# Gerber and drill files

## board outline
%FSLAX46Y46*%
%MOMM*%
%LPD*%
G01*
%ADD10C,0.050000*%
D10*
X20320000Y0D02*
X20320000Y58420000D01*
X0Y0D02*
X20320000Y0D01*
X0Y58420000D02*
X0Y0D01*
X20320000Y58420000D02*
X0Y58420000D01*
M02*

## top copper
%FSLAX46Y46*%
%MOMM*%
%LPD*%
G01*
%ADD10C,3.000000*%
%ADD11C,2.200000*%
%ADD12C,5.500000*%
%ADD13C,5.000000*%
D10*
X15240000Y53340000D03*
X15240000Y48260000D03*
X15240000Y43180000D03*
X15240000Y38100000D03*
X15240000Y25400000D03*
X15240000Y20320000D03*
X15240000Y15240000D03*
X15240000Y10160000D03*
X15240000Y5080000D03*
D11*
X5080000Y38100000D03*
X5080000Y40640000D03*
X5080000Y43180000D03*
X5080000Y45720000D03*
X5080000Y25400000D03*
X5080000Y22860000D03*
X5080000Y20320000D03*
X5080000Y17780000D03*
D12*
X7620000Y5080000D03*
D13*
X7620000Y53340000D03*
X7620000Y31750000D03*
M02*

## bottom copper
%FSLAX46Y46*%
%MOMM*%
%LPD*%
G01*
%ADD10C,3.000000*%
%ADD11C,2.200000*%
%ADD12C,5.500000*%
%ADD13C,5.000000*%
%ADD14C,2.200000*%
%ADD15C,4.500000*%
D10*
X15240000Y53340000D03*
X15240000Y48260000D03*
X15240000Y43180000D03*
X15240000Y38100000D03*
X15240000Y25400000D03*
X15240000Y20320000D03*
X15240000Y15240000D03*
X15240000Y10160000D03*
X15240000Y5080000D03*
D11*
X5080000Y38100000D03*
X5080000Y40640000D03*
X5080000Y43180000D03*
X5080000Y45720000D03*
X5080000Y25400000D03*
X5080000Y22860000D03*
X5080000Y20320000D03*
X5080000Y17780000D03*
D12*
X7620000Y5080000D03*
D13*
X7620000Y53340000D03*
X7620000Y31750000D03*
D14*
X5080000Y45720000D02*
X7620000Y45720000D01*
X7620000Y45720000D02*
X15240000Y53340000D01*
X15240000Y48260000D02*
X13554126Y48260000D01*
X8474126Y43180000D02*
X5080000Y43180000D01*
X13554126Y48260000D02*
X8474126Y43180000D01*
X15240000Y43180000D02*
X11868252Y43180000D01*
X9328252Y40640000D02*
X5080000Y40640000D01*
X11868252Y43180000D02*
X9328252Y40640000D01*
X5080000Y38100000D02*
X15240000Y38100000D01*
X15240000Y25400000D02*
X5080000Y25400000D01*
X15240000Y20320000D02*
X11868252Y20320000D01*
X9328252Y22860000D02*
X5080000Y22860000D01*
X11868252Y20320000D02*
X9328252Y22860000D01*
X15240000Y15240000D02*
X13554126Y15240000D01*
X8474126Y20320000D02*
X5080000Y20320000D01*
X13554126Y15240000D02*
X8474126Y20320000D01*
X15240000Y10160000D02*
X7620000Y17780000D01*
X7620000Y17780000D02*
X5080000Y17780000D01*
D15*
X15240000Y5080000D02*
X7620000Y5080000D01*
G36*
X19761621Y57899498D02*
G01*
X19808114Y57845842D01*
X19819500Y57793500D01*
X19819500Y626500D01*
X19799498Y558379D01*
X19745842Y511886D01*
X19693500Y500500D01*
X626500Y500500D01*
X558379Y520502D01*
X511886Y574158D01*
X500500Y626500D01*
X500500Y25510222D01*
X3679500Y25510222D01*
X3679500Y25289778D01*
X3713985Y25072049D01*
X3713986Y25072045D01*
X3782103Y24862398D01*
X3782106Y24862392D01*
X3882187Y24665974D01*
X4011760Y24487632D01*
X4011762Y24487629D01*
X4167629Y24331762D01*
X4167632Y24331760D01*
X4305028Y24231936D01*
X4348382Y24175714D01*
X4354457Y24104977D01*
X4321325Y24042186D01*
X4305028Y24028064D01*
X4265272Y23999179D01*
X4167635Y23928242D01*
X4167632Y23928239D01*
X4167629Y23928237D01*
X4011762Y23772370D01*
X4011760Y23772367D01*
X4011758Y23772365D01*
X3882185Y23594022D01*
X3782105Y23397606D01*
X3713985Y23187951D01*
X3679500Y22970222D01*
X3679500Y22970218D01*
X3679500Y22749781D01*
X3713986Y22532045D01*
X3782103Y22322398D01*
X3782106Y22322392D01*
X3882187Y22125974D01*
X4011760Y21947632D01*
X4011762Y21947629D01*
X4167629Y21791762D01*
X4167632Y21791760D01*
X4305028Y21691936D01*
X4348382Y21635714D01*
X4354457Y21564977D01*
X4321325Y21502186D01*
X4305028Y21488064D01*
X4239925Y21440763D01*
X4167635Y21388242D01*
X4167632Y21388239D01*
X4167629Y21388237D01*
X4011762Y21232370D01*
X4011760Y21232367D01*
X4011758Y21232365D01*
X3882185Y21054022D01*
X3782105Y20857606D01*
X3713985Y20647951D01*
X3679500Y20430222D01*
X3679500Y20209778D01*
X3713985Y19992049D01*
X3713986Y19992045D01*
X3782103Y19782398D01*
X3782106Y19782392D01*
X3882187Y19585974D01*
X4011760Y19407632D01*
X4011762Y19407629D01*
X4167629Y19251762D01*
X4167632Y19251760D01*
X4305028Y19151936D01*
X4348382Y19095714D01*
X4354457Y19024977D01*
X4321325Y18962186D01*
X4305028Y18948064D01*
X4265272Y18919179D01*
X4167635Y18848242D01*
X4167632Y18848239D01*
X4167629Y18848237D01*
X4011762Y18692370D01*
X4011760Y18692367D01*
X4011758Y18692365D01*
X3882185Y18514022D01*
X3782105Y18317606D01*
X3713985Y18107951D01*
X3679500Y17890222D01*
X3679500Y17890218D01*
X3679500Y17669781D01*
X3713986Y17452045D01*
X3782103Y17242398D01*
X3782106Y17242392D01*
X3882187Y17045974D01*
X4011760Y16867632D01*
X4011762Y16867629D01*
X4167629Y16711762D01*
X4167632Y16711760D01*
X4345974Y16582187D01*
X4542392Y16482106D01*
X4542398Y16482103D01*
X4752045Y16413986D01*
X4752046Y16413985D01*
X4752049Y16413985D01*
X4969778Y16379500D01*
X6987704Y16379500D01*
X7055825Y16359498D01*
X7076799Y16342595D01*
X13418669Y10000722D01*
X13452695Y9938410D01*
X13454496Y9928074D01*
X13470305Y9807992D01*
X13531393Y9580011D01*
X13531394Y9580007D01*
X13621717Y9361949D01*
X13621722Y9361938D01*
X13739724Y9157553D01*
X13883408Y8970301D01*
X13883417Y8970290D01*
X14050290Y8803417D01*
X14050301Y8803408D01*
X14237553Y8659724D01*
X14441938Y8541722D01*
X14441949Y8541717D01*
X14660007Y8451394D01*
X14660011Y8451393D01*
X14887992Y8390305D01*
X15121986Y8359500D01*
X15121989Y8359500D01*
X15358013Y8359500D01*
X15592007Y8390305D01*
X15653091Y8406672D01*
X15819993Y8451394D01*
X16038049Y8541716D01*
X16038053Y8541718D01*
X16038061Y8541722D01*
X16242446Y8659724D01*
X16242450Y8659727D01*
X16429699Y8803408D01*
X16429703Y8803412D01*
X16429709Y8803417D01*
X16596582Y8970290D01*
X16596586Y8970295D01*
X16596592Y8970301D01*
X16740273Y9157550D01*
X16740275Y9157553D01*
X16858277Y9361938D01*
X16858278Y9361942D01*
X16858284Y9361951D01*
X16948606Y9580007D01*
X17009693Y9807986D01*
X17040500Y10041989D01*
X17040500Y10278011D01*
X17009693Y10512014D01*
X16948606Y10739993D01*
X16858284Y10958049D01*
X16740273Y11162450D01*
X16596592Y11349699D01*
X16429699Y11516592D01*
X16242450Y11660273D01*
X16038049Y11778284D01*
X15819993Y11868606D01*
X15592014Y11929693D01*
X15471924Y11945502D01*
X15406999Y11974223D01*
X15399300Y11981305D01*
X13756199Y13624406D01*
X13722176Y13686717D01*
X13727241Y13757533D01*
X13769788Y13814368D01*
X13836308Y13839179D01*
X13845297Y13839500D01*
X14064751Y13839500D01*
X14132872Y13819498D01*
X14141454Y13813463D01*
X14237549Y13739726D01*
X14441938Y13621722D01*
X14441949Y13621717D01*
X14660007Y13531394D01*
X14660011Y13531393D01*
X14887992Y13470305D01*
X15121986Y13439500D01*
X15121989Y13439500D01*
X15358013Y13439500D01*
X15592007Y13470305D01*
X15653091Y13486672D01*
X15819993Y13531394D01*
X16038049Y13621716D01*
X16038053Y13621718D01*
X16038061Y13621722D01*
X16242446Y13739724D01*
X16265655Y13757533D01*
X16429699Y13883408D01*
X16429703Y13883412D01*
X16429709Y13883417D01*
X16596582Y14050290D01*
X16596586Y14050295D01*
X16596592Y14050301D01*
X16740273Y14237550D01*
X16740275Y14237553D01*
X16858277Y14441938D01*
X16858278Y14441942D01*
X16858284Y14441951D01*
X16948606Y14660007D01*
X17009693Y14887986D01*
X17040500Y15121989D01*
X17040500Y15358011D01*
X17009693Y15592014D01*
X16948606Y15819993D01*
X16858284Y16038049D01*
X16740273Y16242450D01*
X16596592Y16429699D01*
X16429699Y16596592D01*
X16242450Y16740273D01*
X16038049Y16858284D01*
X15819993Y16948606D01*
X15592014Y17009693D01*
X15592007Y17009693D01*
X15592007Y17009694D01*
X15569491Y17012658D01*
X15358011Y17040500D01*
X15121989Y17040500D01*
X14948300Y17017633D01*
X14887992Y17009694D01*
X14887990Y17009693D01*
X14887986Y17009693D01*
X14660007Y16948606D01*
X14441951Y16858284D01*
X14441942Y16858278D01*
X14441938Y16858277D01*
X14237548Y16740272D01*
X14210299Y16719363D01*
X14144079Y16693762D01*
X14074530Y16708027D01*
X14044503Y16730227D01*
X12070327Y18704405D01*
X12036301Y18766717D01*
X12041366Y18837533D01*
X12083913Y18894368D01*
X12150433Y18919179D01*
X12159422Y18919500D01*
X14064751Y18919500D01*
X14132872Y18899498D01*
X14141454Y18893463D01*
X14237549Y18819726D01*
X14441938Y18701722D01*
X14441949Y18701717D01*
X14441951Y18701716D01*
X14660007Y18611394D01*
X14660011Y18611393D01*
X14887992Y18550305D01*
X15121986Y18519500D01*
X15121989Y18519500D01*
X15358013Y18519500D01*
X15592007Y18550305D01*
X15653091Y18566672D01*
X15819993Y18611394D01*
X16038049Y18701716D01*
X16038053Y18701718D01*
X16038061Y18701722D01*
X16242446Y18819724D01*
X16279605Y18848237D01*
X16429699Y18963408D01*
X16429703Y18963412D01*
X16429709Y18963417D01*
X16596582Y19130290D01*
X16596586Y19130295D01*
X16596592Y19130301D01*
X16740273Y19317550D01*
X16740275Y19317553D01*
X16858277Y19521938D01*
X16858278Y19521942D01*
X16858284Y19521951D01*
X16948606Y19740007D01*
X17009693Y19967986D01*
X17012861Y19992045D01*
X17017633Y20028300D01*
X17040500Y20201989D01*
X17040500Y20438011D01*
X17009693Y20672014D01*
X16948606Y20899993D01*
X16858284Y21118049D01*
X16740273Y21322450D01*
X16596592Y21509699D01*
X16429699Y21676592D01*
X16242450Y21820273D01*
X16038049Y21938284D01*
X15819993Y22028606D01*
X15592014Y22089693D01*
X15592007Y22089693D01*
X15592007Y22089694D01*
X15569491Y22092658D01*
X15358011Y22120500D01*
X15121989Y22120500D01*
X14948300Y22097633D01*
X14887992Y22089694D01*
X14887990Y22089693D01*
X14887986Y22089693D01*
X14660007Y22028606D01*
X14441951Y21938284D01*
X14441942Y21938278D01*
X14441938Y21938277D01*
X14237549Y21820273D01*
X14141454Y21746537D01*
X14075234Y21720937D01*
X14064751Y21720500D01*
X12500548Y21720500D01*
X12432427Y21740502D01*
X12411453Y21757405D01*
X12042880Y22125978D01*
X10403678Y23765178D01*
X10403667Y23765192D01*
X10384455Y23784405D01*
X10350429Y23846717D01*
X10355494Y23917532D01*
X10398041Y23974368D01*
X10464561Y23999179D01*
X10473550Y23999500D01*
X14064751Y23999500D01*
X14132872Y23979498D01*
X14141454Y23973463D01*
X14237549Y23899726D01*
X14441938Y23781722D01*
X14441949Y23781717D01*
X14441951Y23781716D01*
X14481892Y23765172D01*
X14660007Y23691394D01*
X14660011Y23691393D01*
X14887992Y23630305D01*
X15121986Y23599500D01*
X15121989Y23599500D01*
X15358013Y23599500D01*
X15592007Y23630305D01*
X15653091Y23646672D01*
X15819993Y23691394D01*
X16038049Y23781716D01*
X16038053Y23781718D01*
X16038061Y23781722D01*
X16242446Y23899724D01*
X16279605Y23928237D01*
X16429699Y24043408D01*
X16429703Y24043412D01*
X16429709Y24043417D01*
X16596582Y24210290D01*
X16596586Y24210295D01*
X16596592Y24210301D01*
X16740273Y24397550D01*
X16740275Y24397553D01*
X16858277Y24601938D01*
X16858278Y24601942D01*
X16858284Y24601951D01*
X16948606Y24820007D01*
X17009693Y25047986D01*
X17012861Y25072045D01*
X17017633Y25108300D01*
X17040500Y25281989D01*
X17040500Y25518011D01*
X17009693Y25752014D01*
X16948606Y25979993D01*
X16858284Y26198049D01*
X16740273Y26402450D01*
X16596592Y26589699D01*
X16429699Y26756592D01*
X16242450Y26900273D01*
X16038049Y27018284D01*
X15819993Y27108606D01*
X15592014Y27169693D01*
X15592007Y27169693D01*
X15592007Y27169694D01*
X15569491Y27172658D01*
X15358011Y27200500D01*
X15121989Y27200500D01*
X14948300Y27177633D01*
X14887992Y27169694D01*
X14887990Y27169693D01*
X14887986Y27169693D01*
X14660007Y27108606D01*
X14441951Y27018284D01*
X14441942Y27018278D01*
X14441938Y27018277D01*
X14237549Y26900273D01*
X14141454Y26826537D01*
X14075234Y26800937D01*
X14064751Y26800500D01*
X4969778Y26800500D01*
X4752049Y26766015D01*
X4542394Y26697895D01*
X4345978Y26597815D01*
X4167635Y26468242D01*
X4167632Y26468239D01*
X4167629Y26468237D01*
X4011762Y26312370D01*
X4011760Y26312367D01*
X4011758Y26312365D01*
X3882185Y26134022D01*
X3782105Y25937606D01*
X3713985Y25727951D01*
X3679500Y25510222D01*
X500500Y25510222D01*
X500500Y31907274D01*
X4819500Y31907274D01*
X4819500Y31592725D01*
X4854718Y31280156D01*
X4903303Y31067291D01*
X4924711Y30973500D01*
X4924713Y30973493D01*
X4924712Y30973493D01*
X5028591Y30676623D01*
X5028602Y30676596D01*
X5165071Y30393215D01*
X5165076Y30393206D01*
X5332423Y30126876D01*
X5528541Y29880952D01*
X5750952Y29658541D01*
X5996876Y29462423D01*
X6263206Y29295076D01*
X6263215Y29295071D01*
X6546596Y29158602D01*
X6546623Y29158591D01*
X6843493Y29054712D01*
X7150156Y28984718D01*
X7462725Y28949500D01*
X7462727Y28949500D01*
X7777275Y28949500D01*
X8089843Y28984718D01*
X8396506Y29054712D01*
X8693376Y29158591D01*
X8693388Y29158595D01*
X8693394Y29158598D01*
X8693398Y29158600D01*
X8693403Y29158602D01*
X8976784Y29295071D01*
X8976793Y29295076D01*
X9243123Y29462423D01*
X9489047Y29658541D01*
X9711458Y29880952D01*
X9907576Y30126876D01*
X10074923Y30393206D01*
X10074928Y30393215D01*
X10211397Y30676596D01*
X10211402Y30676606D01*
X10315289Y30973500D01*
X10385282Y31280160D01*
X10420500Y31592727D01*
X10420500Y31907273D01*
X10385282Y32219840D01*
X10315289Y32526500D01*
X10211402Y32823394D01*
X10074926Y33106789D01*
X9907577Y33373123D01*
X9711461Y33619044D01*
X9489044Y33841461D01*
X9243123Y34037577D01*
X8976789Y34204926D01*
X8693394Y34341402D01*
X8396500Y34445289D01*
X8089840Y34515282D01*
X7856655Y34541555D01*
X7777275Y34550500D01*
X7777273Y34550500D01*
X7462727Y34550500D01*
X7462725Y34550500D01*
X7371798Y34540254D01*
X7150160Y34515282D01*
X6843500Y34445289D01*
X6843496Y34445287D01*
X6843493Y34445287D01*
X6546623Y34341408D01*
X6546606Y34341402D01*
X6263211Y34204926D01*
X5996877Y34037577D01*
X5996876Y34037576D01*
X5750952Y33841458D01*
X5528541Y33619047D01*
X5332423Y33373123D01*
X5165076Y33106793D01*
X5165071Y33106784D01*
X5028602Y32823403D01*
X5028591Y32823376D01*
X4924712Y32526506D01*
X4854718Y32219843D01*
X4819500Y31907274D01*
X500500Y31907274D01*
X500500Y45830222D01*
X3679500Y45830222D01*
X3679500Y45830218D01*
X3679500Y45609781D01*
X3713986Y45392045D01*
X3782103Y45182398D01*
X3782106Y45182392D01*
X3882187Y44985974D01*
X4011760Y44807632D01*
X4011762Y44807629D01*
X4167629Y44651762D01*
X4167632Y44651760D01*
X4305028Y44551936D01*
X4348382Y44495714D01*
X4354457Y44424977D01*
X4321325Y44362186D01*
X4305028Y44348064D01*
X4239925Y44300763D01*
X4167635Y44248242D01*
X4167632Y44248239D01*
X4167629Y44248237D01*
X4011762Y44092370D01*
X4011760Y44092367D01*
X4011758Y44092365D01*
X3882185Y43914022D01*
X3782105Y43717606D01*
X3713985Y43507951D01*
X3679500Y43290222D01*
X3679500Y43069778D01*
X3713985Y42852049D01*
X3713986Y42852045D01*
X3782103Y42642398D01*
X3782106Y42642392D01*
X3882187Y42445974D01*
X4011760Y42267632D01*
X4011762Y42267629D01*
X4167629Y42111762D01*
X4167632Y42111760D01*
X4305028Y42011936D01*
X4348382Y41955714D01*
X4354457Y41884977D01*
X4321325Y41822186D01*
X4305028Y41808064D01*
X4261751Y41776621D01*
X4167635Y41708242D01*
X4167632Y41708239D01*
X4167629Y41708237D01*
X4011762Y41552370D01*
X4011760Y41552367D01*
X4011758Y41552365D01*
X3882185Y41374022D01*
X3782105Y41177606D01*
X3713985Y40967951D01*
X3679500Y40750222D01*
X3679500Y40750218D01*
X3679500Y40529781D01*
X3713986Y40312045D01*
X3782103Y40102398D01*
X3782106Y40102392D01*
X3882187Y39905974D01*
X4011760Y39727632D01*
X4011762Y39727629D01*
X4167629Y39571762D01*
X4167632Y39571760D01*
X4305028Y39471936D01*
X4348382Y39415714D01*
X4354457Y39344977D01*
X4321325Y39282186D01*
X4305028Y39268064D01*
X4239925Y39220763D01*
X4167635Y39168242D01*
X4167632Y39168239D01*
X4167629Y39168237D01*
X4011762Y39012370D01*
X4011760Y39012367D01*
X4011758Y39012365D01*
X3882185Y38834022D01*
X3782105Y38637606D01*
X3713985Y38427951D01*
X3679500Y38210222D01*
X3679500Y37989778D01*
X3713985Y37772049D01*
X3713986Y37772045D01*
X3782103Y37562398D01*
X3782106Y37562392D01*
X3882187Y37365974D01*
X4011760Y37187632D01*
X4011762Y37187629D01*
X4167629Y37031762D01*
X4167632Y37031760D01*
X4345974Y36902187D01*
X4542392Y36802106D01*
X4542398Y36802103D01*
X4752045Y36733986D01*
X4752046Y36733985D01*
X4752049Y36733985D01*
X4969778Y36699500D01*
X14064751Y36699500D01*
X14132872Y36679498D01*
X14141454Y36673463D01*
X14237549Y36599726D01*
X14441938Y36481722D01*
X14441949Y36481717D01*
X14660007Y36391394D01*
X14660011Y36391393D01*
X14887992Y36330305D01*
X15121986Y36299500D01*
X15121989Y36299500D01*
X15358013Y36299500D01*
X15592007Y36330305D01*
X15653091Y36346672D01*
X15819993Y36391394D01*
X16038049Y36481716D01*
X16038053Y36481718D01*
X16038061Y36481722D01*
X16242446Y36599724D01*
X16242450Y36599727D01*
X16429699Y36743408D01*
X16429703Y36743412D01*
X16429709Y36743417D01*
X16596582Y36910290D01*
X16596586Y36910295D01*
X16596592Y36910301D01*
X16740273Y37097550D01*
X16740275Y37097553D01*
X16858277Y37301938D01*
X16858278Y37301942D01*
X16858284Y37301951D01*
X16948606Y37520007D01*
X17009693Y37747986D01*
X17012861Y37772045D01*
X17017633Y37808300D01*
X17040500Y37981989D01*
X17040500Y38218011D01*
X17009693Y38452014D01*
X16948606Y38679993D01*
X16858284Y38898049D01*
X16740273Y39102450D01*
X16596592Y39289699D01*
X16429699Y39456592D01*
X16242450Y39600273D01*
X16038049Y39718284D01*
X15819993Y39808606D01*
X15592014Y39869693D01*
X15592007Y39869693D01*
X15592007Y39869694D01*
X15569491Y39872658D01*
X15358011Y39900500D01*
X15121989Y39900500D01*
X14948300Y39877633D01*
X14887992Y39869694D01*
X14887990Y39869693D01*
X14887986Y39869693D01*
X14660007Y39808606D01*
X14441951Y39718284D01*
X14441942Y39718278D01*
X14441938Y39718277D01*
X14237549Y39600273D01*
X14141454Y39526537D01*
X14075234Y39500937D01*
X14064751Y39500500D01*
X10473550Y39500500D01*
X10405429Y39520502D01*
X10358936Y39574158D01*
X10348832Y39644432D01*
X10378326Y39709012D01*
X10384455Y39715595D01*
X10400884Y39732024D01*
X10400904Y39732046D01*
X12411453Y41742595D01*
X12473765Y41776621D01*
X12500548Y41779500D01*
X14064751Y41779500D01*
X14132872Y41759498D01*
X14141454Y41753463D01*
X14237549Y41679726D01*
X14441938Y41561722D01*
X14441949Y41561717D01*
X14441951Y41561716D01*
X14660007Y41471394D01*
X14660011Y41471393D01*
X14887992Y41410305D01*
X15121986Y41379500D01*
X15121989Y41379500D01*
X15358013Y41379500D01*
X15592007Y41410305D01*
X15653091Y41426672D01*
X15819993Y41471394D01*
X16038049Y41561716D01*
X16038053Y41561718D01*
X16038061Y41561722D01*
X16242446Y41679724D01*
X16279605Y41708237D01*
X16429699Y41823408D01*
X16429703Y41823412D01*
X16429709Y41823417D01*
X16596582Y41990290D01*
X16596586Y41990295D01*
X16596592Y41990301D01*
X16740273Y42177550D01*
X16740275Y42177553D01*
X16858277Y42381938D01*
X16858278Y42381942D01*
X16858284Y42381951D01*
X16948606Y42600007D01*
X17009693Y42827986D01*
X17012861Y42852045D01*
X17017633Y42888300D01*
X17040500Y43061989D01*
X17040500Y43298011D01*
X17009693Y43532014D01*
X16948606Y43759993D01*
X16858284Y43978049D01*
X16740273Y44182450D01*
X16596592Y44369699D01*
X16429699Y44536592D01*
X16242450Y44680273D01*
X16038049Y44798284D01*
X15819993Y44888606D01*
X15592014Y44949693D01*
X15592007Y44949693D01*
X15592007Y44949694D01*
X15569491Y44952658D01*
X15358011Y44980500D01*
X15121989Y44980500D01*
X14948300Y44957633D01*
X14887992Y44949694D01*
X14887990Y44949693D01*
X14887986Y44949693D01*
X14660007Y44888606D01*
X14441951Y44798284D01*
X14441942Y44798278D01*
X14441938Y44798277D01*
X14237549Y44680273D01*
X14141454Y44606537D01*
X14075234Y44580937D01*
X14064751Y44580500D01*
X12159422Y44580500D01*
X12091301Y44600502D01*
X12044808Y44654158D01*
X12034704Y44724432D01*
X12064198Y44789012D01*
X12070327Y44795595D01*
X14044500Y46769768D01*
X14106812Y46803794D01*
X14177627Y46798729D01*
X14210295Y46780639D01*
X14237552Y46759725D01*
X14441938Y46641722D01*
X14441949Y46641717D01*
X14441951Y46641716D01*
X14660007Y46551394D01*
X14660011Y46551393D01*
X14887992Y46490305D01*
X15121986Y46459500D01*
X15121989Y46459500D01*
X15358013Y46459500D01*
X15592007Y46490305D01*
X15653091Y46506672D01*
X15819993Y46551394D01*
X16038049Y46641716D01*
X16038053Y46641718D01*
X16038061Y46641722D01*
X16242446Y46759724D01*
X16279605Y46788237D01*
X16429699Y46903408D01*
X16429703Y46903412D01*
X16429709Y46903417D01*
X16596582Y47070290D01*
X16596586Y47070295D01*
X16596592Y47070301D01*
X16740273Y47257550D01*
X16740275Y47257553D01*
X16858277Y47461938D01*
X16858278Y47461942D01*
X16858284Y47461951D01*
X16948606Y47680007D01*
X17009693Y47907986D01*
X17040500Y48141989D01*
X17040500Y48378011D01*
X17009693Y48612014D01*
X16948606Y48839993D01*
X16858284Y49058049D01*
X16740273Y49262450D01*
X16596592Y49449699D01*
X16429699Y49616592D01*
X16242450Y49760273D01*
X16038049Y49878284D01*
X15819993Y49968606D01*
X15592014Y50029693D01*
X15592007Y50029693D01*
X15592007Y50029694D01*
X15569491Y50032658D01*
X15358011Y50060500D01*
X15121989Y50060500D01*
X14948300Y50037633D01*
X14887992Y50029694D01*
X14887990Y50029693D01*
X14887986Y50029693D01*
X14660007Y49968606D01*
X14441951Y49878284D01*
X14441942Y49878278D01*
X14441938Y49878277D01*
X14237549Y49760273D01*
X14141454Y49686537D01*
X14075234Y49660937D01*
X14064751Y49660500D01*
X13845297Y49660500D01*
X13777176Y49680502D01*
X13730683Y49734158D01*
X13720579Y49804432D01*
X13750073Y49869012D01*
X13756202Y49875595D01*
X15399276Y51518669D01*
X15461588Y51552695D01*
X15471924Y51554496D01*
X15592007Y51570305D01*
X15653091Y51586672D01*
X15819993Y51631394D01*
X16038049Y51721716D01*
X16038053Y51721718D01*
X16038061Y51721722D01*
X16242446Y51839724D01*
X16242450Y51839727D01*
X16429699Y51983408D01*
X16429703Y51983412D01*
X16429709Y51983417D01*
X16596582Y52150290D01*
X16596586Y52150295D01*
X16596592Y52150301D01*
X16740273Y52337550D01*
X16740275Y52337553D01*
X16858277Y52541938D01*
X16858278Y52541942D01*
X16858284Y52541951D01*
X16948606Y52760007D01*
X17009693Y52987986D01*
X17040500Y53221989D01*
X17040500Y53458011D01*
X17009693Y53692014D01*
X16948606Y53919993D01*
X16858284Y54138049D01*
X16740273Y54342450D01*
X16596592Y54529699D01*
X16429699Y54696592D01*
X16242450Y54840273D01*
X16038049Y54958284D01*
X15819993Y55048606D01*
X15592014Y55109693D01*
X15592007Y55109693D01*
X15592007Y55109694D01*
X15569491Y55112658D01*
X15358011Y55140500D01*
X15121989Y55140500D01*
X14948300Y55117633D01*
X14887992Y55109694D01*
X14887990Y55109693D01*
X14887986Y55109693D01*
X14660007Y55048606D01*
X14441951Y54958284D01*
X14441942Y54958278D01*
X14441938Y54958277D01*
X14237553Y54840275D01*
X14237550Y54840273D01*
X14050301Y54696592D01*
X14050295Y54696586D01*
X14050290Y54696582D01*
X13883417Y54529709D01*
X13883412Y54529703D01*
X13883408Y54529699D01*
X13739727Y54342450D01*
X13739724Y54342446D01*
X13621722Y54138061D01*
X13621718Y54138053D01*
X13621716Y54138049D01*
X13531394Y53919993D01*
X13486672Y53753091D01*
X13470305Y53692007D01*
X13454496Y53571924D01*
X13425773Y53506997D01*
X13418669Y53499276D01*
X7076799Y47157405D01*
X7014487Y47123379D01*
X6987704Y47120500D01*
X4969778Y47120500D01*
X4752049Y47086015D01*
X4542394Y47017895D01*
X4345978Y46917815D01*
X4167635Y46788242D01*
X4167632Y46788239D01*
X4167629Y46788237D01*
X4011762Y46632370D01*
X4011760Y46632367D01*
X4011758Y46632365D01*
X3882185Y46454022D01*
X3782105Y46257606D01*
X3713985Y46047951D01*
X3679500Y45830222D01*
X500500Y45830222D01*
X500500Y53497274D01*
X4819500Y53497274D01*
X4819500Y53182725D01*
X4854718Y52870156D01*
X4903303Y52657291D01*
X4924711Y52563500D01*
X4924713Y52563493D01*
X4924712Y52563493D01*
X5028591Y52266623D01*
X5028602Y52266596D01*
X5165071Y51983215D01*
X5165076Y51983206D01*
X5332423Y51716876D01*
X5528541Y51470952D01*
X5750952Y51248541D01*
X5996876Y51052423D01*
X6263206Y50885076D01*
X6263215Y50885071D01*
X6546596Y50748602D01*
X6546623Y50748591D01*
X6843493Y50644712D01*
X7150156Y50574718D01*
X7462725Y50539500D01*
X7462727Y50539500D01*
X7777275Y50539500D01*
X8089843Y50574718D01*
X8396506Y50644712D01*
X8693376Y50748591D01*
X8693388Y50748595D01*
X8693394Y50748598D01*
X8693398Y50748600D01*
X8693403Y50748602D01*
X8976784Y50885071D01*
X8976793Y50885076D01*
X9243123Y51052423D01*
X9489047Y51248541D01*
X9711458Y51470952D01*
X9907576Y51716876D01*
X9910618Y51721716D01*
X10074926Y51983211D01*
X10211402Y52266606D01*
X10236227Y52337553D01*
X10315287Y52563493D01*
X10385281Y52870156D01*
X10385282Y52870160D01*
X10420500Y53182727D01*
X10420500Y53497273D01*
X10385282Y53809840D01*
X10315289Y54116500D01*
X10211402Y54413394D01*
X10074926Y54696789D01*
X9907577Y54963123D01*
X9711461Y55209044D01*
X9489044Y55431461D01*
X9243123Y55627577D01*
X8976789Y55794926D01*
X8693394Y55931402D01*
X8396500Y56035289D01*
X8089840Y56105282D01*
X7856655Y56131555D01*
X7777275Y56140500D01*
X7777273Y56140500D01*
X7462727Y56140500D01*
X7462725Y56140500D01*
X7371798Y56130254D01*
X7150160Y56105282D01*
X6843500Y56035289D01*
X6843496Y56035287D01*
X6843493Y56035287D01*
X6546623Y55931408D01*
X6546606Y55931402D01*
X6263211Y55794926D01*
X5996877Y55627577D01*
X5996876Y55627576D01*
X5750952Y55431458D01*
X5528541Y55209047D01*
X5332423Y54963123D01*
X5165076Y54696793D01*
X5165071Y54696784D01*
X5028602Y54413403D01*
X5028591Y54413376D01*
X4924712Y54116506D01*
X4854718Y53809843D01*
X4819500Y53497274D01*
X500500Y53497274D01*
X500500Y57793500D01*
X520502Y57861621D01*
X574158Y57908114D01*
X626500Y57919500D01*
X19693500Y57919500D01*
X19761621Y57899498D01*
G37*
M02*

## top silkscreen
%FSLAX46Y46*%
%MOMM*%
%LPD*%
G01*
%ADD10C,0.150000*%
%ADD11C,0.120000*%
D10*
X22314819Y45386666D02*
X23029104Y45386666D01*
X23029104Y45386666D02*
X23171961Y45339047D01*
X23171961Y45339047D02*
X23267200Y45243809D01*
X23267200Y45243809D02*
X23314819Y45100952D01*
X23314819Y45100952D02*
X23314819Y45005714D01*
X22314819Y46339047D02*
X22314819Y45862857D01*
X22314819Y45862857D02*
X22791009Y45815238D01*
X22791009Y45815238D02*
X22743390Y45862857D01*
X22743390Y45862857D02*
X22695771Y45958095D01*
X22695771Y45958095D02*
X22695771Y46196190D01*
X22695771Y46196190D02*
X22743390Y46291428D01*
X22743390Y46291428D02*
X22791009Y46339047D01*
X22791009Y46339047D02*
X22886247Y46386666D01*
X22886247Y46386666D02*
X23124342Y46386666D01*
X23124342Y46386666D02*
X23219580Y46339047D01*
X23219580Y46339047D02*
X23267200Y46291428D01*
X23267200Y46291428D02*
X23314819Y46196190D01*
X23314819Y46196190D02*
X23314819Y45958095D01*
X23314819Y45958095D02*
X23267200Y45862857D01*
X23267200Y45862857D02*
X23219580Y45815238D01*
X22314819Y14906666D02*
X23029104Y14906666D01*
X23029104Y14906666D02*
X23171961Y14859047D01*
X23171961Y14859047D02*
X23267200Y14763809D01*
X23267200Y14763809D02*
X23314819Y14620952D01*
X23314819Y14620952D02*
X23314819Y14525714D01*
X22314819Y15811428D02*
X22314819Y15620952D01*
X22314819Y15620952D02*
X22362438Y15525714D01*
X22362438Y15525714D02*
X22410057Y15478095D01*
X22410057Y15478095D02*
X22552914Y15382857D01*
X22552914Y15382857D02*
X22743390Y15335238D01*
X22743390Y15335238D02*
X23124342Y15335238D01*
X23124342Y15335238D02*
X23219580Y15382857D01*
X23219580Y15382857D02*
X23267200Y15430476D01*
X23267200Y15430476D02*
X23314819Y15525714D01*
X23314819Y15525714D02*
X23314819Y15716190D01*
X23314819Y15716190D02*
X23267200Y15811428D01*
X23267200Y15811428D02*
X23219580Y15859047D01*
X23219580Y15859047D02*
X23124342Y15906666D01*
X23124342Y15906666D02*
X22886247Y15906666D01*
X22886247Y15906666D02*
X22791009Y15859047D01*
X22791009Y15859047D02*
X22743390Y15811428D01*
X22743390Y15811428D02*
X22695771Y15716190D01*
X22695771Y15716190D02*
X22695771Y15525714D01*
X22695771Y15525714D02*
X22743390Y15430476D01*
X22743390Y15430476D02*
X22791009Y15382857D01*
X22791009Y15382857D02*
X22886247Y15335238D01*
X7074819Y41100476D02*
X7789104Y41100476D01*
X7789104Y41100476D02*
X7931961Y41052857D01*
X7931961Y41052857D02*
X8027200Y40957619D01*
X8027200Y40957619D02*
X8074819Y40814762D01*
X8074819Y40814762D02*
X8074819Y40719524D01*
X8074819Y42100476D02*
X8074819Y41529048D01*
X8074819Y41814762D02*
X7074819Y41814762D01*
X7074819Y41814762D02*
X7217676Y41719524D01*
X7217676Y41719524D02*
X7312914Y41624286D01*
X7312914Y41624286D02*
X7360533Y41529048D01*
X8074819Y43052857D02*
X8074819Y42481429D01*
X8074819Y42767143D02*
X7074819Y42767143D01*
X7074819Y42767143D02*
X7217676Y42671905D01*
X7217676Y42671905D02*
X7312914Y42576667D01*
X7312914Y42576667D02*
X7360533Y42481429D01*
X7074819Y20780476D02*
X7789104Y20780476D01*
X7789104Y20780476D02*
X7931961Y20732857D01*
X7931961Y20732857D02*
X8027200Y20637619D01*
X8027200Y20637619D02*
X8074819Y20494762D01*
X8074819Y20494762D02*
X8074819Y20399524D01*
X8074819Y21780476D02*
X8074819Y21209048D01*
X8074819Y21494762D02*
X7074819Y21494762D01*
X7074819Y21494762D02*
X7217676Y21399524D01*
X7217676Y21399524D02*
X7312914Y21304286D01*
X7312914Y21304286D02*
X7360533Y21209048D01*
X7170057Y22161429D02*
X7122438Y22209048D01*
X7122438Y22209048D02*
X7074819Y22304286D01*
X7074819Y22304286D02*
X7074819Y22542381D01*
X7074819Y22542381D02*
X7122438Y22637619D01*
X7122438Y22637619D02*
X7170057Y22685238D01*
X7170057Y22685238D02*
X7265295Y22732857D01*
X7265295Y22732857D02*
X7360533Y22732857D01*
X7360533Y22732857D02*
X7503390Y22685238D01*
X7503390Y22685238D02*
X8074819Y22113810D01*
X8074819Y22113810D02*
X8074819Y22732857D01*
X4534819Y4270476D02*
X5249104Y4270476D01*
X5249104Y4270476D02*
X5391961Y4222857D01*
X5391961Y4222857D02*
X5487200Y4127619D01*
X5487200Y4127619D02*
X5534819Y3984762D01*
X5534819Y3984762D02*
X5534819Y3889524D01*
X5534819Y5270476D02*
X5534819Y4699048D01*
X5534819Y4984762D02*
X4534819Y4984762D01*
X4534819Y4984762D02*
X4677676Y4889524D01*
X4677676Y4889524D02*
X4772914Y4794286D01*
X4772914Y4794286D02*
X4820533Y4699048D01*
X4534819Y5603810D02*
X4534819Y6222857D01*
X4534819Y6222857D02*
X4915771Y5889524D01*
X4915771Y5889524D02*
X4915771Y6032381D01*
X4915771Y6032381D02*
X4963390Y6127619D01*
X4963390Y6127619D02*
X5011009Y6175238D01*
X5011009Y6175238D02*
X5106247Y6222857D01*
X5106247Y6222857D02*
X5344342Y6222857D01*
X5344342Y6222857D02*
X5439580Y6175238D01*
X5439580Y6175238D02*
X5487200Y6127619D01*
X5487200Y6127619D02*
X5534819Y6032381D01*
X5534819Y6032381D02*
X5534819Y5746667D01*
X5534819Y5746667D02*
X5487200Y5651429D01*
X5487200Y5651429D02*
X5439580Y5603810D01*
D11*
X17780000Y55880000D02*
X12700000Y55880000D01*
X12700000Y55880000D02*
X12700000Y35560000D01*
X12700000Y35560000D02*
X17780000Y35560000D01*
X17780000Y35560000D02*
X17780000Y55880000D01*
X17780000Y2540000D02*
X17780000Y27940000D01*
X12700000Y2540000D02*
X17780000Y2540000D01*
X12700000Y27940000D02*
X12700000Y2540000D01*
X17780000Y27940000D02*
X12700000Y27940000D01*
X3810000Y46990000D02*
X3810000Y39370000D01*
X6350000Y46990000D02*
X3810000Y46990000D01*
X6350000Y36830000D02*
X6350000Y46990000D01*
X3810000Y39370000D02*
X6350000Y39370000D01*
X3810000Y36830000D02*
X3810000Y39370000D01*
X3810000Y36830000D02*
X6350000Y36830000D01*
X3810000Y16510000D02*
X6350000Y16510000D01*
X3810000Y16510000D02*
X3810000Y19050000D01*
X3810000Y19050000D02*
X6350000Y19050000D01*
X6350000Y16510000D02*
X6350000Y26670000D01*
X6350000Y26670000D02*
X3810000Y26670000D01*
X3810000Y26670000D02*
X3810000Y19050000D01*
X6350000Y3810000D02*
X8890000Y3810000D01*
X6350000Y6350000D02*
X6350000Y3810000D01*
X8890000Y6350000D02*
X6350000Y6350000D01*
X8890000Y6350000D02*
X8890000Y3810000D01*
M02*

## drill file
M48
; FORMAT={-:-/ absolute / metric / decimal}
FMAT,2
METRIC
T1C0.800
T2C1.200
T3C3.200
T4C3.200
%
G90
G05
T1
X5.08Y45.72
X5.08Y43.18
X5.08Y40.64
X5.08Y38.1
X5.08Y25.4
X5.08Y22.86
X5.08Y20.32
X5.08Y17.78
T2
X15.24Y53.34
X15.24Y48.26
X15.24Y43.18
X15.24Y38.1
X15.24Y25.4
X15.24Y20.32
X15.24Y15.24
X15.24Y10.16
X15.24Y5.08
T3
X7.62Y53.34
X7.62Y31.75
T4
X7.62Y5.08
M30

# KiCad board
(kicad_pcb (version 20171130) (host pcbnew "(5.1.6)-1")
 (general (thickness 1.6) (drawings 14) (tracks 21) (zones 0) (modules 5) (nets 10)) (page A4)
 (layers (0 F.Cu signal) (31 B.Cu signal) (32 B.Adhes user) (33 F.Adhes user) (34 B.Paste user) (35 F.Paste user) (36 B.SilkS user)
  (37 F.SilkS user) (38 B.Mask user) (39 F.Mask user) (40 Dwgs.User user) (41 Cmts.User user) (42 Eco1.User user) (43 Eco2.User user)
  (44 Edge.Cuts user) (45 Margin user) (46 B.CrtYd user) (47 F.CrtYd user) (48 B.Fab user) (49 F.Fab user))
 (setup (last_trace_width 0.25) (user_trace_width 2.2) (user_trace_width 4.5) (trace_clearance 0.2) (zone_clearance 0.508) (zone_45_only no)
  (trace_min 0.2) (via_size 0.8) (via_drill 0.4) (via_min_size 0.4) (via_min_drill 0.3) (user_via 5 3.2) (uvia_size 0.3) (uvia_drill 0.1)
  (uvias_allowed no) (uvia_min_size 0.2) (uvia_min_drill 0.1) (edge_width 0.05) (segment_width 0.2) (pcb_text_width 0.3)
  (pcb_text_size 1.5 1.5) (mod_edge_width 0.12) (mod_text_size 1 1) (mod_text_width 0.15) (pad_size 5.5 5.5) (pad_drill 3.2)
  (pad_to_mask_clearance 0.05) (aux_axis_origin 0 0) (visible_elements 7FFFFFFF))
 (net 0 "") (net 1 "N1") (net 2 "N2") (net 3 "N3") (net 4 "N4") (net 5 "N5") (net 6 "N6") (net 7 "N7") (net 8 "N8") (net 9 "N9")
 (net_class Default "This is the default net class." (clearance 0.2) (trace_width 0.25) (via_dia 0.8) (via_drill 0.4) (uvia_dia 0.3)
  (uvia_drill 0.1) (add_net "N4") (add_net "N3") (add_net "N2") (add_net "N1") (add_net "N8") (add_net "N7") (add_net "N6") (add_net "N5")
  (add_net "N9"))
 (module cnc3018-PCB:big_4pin (layer F.Cu) (at 15.24 -45.72 270)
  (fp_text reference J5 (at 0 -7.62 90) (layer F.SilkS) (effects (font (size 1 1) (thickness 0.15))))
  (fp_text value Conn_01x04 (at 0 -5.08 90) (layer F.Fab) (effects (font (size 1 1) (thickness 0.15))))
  (fp_line (start -10.16 -2.54) (end -10.16 2.54) (layer F.SilkS) (width 0.12))
  (fp_line (start -10.16 2.54) (end 10.16 2.54) (layer F.SilkS) (width 0.12))
  (fp_line (start 10.16 2.54) (end 10.16 -2.54) (layer F.SilkS) (width 0.12))
  (fp_line (start 10.16 -2.54) (end -10.16 -2.54) (layer F.SilkS) (width 0.12))
  (pad 1 thru_hole circle (at -7.62 0 270) (size 3 3) (drill 1.2) (layers *.Cu *.Mask) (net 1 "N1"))
  (pad 2 thru_hole circle (at -2.54 0 270) (size 3 3) (drill 1.2) (layers *.Cu *.Mask) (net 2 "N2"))
  (pad 3 thru_hole circle (at 2.54 0 270) (size 3 3) (drill 1.2) (layers *.Cu *.Mask) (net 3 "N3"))
  (pad 4 thru_hole circle (at 7.62 0 270) (size 3 3) (drill 1.2) (layers *.Cu *.Mask) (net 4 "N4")))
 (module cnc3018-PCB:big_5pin (layer F.Cu) (at 15.24 -15.24 270)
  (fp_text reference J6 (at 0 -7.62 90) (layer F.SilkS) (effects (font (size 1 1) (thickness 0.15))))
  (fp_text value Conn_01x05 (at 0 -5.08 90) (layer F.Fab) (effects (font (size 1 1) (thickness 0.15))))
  (fp_line (start 12.7 -2.54) (end -12.7 -2.54) (layer F.SilkS) (width 0.12))
  (fp_line (start 12.7 2.54) (end 12.7 -2.54) (layer F.SilkS) (width 0.12))
  (fp_line (start -12.7 2.54) (end 12.7 2.54) (layer F.SilkS) (width 0.12))
  (fp_line (start -12.7 -2.54) (end -12.7 2.54) (layer F.SilkS) (width 0.12))
  (pad 1 thru_hole circle (at -10.16 0 270) (size 3 3) (drill 1.2) (layers *.Cu *.Mask) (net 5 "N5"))
  (pad 2 thru_hole circle (at -5.08 0 270) (size 3 3) (drill 1.2) (layers *.Cu *.Mask) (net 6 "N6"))
  (pad 3 thru_hole circle (at 0 0 270) (size 3 3) (drill 1.2) (layers *.Cu *.Mask) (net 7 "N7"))
  (pad 4 thru_hole circle (at 5.08 0 270) (size 3 3) (drill 1.2) (layers *.Cu *.Mask) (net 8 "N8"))
  (pad 5 thru_hole circle (at 10.16 0 270) (size 3 3) (drill 1.2) (layers *.Cu *.Mask) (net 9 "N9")))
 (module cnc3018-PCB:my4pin (layer F.Cu) (at 5.08 -38.1 90)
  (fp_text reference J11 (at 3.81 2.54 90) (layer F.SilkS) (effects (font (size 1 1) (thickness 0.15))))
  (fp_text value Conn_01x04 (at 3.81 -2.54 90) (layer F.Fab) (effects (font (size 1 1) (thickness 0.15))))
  (fp_line (start 8.89 -1.27) (end 1.27 -1.27) (layer F.SilkS) (width 0.12))
  (fp_line (start 8.89 1.27) (end 8.89 -1.27) (layer F.SilkS) (width 0.12))
  (fp_line (start -1.27 1.27) (end 8.89 1.27) (layer F.SilkS) (width 0.12))
  (fp_line (start 1.27 -1.27) (end 1.27 1.27) (layer F.SilkS) (width 0.12))
  (fp_line (start -1.27 -1.27) (end 1.27 -1.27) (layer F.SilkS) (width 0.12))
  (fp_line (start -1.27 -1.27) (end -1.27 1.27) (layer F.SilkS) (width 0.12))
  (pad 1 thru_hole circle (at 0 0 90) (size 2.2 2.2) (drill 0.8) (layers *.Cu *.Mask) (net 4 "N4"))
  (pad 2 thru_hole circle (at 2.54 0 90) (size 2.2 2.2) (drill 0.8) (layers *.Cu *.Mask) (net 3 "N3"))
  (pad 3 thru_hole circle (at 5.08 0 90) (size 2.2 2.2) (drill 0.8) (layers *.Cu *.Mask) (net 2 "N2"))
  (pad 4 thru_hole circle (at 7.62 0 90) (size 2.2 2.2) (drill 0.8) (layers *.Cu *.Mask) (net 1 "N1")))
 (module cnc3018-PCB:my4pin (layer F.Cu) (at 5.08 -17.78 90)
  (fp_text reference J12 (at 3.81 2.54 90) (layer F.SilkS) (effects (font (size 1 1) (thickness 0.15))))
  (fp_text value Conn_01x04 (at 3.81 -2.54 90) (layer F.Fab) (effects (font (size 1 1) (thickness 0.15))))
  (fp_line (start -1.27 -1.27) (end -1.27 1.27) (layer F.SilkS) (width 0.12))
  (fp_line (start -1.27 -1.27) (end 1.27 -1.27) (layer F.SilkS) (width 0.12))
  (fp_line (start 1.27 -1.27) (end 1.27 1.27) (layer F.SilkS) (width 0.12))
  (fp_line (start -1.27 1.27) (end 8.89 1.27) (layer F.SilkS) (width 0.12))
  (fp_line (start 8.89 1.27) (end 8.89 -1.27) (layer F.SilkS) (width 0.12))
  (fp_line (start 8.89 -1.27) (end 1.27 -1.27) (layer F.SilkS) (width 0.12))
  (pad 4 thru_hole circle (at 7.62 0 90) (size 2.2 2.2) (drill 0.8) (layers *.Cu *.Mask) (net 5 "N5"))
  (pad 3 thru_hole circle (at 5.08 0 90) (size 2.2 2.2) (drill 0.8) (layers *.Cu *.Mask) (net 6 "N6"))
  (pad 2 thru_hole circle (at 2.54 0 90) (size 2.2 2.2) (drill 0.8) (layers *.Cu *.Mask) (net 7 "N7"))
  (pad 1 thru_hole circle (at 0 0 90) (size 2.2 2.2) (drill 0.8) (layers *.Cu *.Mask) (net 8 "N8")))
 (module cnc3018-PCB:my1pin (layer F.Cu) (at 7.62 -5.08 270)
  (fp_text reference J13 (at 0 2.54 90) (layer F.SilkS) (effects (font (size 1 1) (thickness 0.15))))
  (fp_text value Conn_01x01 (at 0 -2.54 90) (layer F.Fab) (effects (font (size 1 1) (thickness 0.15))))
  (fp_line (start 1.27 1.27) (end 1.27 -1.27) (layer F.SilkS) (width 0.12))
  (fp_line (start -1.27 1.27) (end 1.27 1.27) (layer F.SilkS) (width 0.12))
  (fp_line (start -1.27 -1.27) (end -1.27 1.27) (layer F.SilkS) (width 0.12))
  (fp_line (start -1.27 -1.27) (end 1.27 -1.27) (layer F.SilkS) (width 0.12))
  (pad 1 thru_hole circle (at 0 0 270) (size 5.5 5.5) (drill 3.2) (layers *.Cu *.Mask) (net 9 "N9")))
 (gr_line (start 20.32 0) (end 20.32 -58.42) (layer Edge.Cuts) (width 0.05))
 (gr_line (start 0 0) (end 20.32 0) (layer Edge.Cuts) (width 0.05))
 (gr_line (start 0 -58.42) (end 0 0) (layer Edge.Cuts) (width 0.05))
 (gr_line (start 20.32 -58.42) (end 0 -58.42) (layer Edge.Cuts) (width 0.05))
 (via (at 7.62 -53.34) (size 5) (drill 3.2) (layers F.Cu B.Cu) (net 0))
 (via (at 7.62 -31.75) (size 5) (drill 3.2) (layers F.Cu B.Cu) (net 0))
 (segment (start 5.08 -45.72) (end 7.62 -45.72) (width 2.2) (layer B.Cu) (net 1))
 (segment (start 7.62 -45.72) (end 15.24 -53.34) (width 2.2) (layer B.Cu) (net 1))
 (segment (start 15.24 -48.26) (end 13.554126 -48.26) (width 2.2) (layer B.Cu) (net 2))
 (segment (start 8.474126 -43.18) (end 5.08 -43.18) (width 2.2) (layer B.Cu) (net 2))
 (segment (start 13.554126 -48.26) (end 8.474126 -43.18) (width 2.2) (layer B.Cu) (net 2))
 (segment (start 15.24 -43.18) (end 11.868252 -43.18) (width 2.2) (layer B.Cu) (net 3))
 (segment (start 9.328252 -40.64) (end 5.08 -40.64) (width 2.2) (layer B.Cu) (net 3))
 (segment (start 11.868252 -43.18) (end 9.328252 -40.64) (width 2.2) (layer B.Cu) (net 3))
 (segment (start 5.08 -38.1) (end 15.24 -38.1) (width 2.2) (layer B.Cu) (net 4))
 (segment (start 15.24 -25.4) (end 5.08 -25.4) (width 2.2) (layer B.Cu) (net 5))
 (segment (start 15.24 -20.32) (end 11.868252 -20.32) (width 2.2) (layer B.Cu) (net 6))
 (segment (start 9.328252 -22.86) (end 5.08 -22.86) (width 2.2) (layer B.Cu) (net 6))
 (segment (start 11.868252 -20.32) (end 9.328252 -22.86) (width 2.2) (layer B.Cu) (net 6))
 (segment (start 15.24 -15.24) (end 13.554126 -15.24) (width 2.2) (layer B.Cu) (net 7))
 (segment (start 8.474126 -20.32) (end 5.08 -20.32) (width 2.2) (layer B.Cu) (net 7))
 (segment (start 13.554126 -15.24) (end 8.474126 -20.32) (width 2.2) (layer B.Cu) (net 7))
 (segment (start 15.24 -10.16) (end 7.62 -17.78) (width 2.2) (layer B.Cu) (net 8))
 (segment (start 7.62 -17.78) (end 5.08 -17.78) (width 2.2) (layer B.Cu) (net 8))
 (segment (start 15.24 -5.08) (end 7.62 -5.08) (width 4.5) (layer B.Cu) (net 9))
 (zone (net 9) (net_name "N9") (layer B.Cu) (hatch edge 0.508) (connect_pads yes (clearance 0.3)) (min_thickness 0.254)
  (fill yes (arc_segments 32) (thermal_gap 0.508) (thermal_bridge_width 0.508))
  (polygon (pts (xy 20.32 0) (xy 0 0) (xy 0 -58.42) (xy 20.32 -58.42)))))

